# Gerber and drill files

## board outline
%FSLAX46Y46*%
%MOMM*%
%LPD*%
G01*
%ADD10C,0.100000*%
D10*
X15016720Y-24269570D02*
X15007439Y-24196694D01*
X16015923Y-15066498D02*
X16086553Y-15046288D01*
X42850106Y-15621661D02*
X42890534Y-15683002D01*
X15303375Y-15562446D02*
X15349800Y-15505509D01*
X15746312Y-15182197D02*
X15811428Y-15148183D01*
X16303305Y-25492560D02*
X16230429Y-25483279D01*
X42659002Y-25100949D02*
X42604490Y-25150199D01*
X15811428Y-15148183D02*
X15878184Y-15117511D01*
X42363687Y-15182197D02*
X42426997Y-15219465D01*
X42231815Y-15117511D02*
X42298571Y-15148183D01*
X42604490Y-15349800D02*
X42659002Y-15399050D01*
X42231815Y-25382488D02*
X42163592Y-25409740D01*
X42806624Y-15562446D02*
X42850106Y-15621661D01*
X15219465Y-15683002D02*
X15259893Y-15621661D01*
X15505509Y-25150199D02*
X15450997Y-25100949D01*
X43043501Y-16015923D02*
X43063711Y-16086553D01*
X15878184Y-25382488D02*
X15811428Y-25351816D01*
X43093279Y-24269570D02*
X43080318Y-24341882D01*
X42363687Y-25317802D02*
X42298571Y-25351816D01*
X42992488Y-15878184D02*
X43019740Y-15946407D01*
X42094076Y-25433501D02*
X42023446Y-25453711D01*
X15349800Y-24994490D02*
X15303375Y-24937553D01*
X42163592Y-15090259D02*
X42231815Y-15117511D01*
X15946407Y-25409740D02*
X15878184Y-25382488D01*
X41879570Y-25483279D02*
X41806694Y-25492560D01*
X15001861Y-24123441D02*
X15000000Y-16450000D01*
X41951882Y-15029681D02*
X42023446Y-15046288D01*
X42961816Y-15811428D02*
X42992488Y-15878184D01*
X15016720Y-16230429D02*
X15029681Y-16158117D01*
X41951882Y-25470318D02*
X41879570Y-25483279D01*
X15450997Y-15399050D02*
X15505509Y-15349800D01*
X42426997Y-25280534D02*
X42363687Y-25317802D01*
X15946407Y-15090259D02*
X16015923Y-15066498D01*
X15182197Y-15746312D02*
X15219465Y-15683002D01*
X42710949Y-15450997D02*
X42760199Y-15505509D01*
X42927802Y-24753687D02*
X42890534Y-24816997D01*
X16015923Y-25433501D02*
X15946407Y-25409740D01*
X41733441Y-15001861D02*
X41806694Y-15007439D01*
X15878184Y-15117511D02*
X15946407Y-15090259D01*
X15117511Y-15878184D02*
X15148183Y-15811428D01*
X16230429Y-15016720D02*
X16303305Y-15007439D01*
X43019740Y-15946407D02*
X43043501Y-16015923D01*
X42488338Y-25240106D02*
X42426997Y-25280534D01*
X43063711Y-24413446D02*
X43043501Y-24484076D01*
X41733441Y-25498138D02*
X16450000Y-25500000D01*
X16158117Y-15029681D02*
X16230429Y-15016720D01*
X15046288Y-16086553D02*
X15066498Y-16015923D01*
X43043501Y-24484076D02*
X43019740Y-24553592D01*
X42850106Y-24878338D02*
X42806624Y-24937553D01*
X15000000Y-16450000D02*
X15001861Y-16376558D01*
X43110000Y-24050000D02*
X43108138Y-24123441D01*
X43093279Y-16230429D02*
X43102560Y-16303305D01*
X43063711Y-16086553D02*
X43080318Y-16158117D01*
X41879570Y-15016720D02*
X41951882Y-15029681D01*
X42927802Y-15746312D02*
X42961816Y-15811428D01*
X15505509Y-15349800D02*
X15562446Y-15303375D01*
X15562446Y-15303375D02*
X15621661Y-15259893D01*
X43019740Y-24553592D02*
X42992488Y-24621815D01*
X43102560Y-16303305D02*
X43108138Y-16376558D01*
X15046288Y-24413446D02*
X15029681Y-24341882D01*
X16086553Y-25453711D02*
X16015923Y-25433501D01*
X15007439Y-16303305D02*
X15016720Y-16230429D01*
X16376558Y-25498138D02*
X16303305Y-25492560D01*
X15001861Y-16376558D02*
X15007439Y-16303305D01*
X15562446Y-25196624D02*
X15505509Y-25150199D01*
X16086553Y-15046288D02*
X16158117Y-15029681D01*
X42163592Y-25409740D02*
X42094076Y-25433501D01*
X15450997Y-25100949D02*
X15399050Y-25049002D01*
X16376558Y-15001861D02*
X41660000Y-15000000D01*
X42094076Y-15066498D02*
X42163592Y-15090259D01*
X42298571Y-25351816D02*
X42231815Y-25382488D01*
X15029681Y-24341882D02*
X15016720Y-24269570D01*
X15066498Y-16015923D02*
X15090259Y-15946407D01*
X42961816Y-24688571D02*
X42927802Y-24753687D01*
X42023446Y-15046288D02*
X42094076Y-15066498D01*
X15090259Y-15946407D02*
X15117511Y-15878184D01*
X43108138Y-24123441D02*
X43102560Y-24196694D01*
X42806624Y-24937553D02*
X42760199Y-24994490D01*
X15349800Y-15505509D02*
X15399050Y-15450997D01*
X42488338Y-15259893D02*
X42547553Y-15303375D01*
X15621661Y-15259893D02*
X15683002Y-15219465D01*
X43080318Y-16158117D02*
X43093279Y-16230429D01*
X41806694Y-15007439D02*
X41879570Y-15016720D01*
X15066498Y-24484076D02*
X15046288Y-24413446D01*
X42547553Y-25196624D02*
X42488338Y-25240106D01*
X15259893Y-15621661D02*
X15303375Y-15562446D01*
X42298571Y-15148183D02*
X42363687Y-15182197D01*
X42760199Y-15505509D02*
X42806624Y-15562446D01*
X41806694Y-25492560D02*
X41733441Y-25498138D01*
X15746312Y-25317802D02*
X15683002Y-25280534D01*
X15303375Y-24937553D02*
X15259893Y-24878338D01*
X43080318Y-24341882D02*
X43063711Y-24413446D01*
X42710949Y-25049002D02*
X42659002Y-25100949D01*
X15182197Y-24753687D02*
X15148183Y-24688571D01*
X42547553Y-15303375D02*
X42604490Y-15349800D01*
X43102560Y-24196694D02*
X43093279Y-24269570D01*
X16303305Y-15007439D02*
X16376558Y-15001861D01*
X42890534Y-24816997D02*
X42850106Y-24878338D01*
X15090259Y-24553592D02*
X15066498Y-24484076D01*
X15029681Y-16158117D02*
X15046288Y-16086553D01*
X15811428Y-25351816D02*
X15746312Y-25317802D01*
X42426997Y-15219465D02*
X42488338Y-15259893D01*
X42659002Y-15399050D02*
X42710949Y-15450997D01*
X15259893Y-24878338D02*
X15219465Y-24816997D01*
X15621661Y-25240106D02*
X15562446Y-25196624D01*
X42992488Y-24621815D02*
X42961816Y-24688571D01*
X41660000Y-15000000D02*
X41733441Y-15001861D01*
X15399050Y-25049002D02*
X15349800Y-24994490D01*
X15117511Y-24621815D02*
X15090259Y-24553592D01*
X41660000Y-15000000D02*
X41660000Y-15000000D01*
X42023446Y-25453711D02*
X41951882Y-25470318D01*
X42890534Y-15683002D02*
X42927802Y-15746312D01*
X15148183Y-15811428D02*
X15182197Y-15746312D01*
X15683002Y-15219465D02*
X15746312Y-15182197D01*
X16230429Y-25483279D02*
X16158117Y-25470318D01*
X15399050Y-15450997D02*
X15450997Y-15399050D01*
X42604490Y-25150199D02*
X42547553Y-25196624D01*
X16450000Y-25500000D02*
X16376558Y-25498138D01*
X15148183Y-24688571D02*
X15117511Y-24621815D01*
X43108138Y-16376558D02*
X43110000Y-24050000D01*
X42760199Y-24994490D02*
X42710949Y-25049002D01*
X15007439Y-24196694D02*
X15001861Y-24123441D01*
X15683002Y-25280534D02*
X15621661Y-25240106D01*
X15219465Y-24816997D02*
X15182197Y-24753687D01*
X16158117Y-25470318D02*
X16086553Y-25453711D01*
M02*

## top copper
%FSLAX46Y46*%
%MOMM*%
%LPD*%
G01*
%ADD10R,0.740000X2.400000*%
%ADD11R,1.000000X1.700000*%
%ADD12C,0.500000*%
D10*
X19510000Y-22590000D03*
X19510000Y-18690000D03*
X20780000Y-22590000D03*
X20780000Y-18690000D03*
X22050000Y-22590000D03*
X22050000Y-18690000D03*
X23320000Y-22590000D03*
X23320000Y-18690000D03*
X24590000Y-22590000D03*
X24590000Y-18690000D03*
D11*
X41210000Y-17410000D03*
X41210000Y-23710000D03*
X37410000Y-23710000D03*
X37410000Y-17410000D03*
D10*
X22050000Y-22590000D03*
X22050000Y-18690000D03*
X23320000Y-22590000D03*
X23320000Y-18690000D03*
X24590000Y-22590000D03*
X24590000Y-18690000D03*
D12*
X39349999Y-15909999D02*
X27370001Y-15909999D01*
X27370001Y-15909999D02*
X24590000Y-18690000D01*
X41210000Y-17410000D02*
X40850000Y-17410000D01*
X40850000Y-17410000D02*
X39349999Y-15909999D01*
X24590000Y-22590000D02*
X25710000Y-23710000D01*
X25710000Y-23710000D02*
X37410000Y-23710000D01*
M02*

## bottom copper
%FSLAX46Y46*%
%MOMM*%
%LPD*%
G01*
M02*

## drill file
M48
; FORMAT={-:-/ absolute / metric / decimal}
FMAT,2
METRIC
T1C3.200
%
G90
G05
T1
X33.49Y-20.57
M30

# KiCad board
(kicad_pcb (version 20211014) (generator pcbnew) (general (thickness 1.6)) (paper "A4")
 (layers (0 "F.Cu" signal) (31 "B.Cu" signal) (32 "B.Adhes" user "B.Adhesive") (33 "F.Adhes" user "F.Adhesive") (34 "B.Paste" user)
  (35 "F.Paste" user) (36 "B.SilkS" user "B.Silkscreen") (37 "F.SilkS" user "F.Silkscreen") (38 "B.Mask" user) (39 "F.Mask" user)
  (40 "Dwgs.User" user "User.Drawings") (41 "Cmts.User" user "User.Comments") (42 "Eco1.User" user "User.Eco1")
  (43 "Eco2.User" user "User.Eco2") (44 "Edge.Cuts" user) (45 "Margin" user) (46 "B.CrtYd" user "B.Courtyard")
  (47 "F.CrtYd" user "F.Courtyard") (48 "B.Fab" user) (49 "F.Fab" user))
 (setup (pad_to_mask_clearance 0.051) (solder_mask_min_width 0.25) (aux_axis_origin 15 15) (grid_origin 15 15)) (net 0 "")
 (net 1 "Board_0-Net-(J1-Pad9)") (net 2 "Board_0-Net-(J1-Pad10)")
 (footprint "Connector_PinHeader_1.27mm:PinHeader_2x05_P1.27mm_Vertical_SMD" (layer "F.Cu") (at 22.05 20.64 90)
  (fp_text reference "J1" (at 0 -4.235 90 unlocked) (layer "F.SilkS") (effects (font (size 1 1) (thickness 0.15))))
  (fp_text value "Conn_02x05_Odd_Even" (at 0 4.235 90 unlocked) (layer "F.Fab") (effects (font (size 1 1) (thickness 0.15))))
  (pad "1" smd rect locked (at -1.95 -2.54 90) (size 2.4 0.74) (layers "F.Cu" "F.Paste" "F.Mask"))
  (pad "2" smd rect locked (at 1.95 -2.54 90) (size 2.4 0.74) (layers "F.Cu" "F.Paste" "F.Mask"))
  (pad "3" smd rect locked (at -1.95 -1.27 90) (size 2.4 0.74) (layers "F.Cu" "F.Paste" "F.Mask"))
  (pad "4" smd rect locked (at 1.95 -1.27 90) (size 2.4 0.74) (layers "F.Cu" "F.Paste" "F.Mask"))
  (pad "5" smd rect locked (at -1.95 0 90) (size 2.4 0.74) (layers "F.Cu" "F.Paste" "F.Mask"))
  (pad "6" smd rect locked (at 1.95 0 90) (size 2.4 0.74) (layers "F.Cu" "F.Paste" "F.Mask"))
  (pad "7" smd rect locked (at -1.95 1.27 90) (size 2.4 0.74) (layers "F.Cu" "F.Paste" "F.Mask"))
  (pad "8" smd rect locked (at 1.95 1.27 90) (size 2.4 0.74) (layers "F.Cu" "F.Paste" "F.Mask"))
  (pad "9" smd rect locked (at -1.95 2.54 90) (size 2.4 0.74) (layers "F.Cu" "F.Paste" "F.Mask") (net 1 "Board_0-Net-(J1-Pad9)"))
  (pad "10" smd rect locked (at 1.95 2.54 90) (size 2.4 0.74) (layers "F.Cu" "F.Paste" "F.Mask") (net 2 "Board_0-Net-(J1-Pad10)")))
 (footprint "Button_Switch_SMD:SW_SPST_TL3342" (layer "F.Cu") (at 39.31 20.56 -90)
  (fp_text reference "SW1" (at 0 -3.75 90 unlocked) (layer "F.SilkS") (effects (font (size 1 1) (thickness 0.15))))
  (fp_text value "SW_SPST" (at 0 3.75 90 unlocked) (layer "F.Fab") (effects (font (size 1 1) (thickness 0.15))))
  (pad "1" smd rect locked (at -3.15 -1.9 270) (size 1.7 1) (layers "F.Cu" "F.Paste" "F.Mask") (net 2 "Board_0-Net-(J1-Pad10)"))
  (pad "1" smd rect locked (at 3.15 -1.9 270) (size 1.7 1) (layers "F.Cu" "F.Paste" "F.Mask") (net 2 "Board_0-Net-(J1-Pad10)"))
  (pad "2" smd rect locked (at 3.15 1.9 270) (size 1.7 1) (layers "F.Cu" "F.Paste" "F.Mask") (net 1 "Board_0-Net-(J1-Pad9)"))
  (pad "2" smd rect locked (at -3.15 1.9 270) (size 1.7 1) (layers "F.Cu" "F.Paste" "F.Mask") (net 1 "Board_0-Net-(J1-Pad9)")))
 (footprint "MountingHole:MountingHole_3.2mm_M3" (layer "F.Cu") (at 33.35 20.57 -90)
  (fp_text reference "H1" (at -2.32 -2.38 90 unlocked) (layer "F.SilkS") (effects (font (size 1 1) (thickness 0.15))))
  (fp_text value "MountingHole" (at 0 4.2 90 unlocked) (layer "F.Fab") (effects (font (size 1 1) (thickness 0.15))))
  (pad "" np_thru_hole circle locked (at 0 -0.14 270) (size 3.2 3.2) (drill 3.2) (layers *.Cu *.Mask)))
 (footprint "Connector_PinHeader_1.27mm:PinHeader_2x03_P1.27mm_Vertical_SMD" (layer "F.Cu") (at 23.32 20.64 90)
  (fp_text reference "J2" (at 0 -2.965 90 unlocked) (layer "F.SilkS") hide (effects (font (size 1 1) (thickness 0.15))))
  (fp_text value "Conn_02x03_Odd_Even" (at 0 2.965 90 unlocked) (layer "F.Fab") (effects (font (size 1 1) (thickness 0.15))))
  (pad "1" smd rect locked (at -1.95 -1.27 90) (size 2.4 0.74) (layers "F.Cu" "F.Paste" "F.Mask"))
  (pad "2" smd rect locked (at 1.95 -1.27 90) (size 2.4 0.74) (layers "F.Cu" "F.Paste" "F.Mask"))
  (pad "3" smd rect locked (at -1.95 0 90) (size 2.4 0.74) (layers "F.Cu" "F.Paste" "F.Mask"))
  (pad "4" smd rect locked (at 1.95 0 90) (size 2.4 0.74) (layers "F.Cu" "F.Paste" "F.Mask"))
  (pad "5" smd rect locked (at -1.95 1.27 90) (size 2.4 0.74) (layers "F.Cu" "F.Paste" "F.Mask") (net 1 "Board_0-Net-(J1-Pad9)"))
  (pad "6" smd rect locked (at 1.95 1.27 90) (size 2.4 0.74) (layers "F.Cu" "F.Paste" "F.Mask") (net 2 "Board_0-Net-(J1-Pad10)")))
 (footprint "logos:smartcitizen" (layer "B.Cu") (at 39.49 20.93)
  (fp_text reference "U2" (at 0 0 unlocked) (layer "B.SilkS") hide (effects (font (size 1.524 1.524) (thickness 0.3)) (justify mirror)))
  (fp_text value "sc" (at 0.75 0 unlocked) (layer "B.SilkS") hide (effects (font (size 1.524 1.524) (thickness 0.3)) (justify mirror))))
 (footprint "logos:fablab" (layer "B.Cu") (at 23.85 16.37)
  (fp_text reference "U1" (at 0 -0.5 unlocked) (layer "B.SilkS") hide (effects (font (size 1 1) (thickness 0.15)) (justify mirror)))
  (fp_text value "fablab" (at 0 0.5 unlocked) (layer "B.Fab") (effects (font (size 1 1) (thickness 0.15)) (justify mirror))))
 (gr_line (start 15.01672 24.26957) (end 15.007439 24.196694) (layer "Edge.Cuts") (width 0.1))
 (gr_line (start 16.015923 15.066498) (end 16.086553 15.046288) (layer "Edge.Cuts") (width 0.1))
 (gr_line (start 42.850106 15.621661) (end 42.890534 15.683002) (layer "Edge.Cuts") (width 0.1))
 (gr_line (start 15.303375 15.562446) (end 15.3498 15.505509) (layer "Edge.Cuts") (width 0.1))
 (gr_line (start 15.746312 15.182197) (end 15.811428 15.148183) (layer "Edge.Cuts") (width 0.1))
 (gr_line (start 16.303305 25.49256) (end 16.230429 25.483279) (layer "Edge.Cuts") (width 0.1))
 (gr_line (start 42.659002 25.100949) (end 42.60449 25.150199) (layer "Edge.Cuts") (width 0.1))
 (gr_line (start 15.811428 15.148183) (end 15.878184 15.117511) (layer "Edge.Cuts") (width 0.1))
 (gr_line (start 42.363687 15.182197) (end 42.426997 15.219465) (layer "Edge.Cuts") (width 0.1))
 (gr_line (start 42.231815 15.117511) (end 42.298571 15.148183) (layer "Edge.Cuts") (width 0.1))
 (gr_line (start 42.60449 15.3498) (end 42.659002 15.39905) (layer "Edge.Cuts") (width 0.1))
 (gr_line (start 42.231815 25.382488) (end 42.163592 25.40974) (layer "Edge.Cuts") (width 0.1))
 (gr_line (start 42.806624 15.562446) (end 42.850106 15.621661) (layer "Edge.Cuts") (width 0.1))
 (gr_line (start 15.219465 15.683002) (end 15.259893 15.621661) (layer "Edge.Cuts") (width 0.1))
 (gr_line (start 15.505509 25.150199) (end 15.450997 25.100949) (layer "Edge.Cuts") (width 0.1))
 (gr_line (start 43.043501 16.015923) (end 43.063711 16.086553) (layer "Edge.Cuts") (width 0.1))
 (gr_line (start 15.878184 25.382488) (end 15.811428 25.351816) (layer "Edge.Cuts") (width 0.1))
 (gr_line (start 43.093279 24.26957) (end 43.080318 24.341882) (layer "Edge.Cuts") (width 0.1))
 (gr_line (start 42.363687 25.317802) (end 42.298571 25.351816) (layer "Edge.Cuts") (width 0.1))
 (gr_line (start 42.992488 15.878184) (end 43.01974 15.946407) (layer "Edge.Cuts") (width 0.1))
 (gr_line (start 42.094076 25.433501) (end 42.023446 25.453711) (layer "Edge.Cuts") (width 0.1))
 (gr_line (start 15.3498 24.99449) (end 15.303375 24.937553) (layer "Edge.Cuts") (width 0.1))
 (gr_line (start 42.163592 15.090259) (end 42.231815 15.117511) (layer "Edge.Cuts") (width 0.1))
 (gr_line (start 15.946407 25.40974) (end 15.878184 25.382488) (layer "Edge.Cuts") (width 0.1))
 (gr_line (start 41.87957 25.483279) (end 41.806694 25.49256) (layer "Edge.Cuts") (width 0.1))
 (gr_line (start 15.001861 24.123441) (end 15 16.45) (layer "Edge.Cuts") (width 0.1))
 (gr_line (start 41.951882 15.029681) (end 42.023446 15.046288) (layer "Edge.Cuts") (width 0.1))
 (gr_line (start 42.961816 15.811428) (end 42.992488 15.878184) (layer "Edge.Cuts") (width 0.1))
 (gr_line (start 15.01672 16.230429) (end 15.029681 16.158117) (layer "Edge.Cuts") (width 0.1))
 (gr_line (start 41.951882 25.470318) (end 41.87957 25.483279) (layer "Edge.Cuts") (width 0.1))
 (gr_line (start 15.450997 15.39905) (end 15.505509 15.3498) (layer "Edge.Cuts") (width 0.1))
 (gr_line (start 42.426997 25.280534) (end 42.363687 25.317802) (layer "Edge.Cuts") (width 0.1))
 (gr_line (start 15.946407 15.090259) (end 16.015923 15.066498) (layer "Edge.Cuts") (width 0.1))
 (gr_line (start 15.182197 15.746312) (end 15.219465 15.683002) (layer "Edge.Cuts") (width 0.1))
 (gr_line (start 42.710949 15.450997) (end 42.760199 15.505509) (layer "Edge.Cuts") (width 0.1))
 (gr_line (start 42.927802 24.753687) (end 42.890534 24.816997) (layer "Edge.Cuts") (width 0.1))
 (gr_line (start 16.015923 25.433501) (end 15.946407 25.40974) (layer "Edge.Cuts") (width 0.1))
 (gr_line (start 41.733441 15.001861) (end 41.806694 15.007439) (layer "Edge.Cuts") (width 0.1))
 (gr_line (start 15.878184 15.117511) (end 15.946407 15.090259) (layer "Edge.Cuts") (width 0.1))
 (gr_line (start 15.117511 15.878184) (end 15.148183 15.811428) (layer "Edge.Cuts") (width 0.1))
 (gr_line (start 16.230429 15.01672) (end 16.303305 15.007439) (layer "Edge.Cuts") (width 0.1))
 (gr_line (start 43.01974 15.946407) (end 43.043501 16.015923) (layer "Edge.Cuts") (width 0.1))
 (gr_line (start 42.488338 25.240106) (end 42.426997 25.280534) (layer "Edge.Cuts") (width 0.1))
 (gr_line (start 43.063711 24.413446) (end 43.043501 24.484076) (layer "Edge.Cuts") (width 0.1))
 (gr_line (start 41.733441 25.498138) (end 16.45 25.5) (layer "Edge.Cuts") (width 0.1))
 (gr_line (start 16.158117 15.029681) (end 16.230429 15.01672) (layer "Edge.Cuts") (width 0.1))
 (gr_line (start 15.046288 16.086553) (end 15.066498 16.015923) (layer "Edge.Cuts") (width 0.1))
 (gr_line (start 43.043501 24.484076) (end 43.01974 24.553592) (layer "Edge.Cuts") (width 0.1))
 (gr_line (start 42.850106 24.878338) (end 42.806624 24.937553) (layer "Edge.Cuts") (width 0.1))
 (gr_line (start 15 16.45) (end 15.001861 16.376558) (layer "Edge.Cuts") (width 0.1))
 (gr_line (start 43.11 24.05) (end 43.108138 24.123441) (layer "Edge.Cuts") (width 0.1))
 (gr_line (start 43.093279 16.230429) (end 43.10256 16.303305) (layer "Edge.Cuts") (width 0.1))
 (gr_line (start 43.063711 16.086553) (end 43.080318 16.158117) (layer "Edge.Cuts") (width 0.1))
 (gr_line (start 41.87957 15.01672) (end 41.951882 15.029681) (layer "Edge.Cuts") (width 0.1))
 (gr_line (start 42.927802 15.746312) (end 42.961816 15.811428) (layer "Edge.Cuts") (width 0.1))
 (gr_line (start 15.505509 15.3498) (end 15.562446 15.303375) (layer "Edge.Cuts") (width 0.1))
 (gr_line (start 15.562446 15.303375) (end 15.621661 15.259893) (layer "Edge.Cuts") (width 0.1))
 (gr_line (start 43.01974 24.553592) (end 42.992488 24.621815) (layer "Edge.Cuts") (width 0.1))
 (gr_line (start 43.10256 16.303305) (end 43.108138 16.376558) (layer "Edge.Cuts") (width 0.1))
 (gr_line (start 15.046288 24.413446) (end 15.029681 24.341882) (layer "Edge.Cuts") (width 0.1))
 (gr_line (start 16.086553 25.453711) (end 16.015923 25.433501) (layer "Edge.Cuts") (width 0.1))
 (gr_line (start 15.007439 16.303305) (end 15.01672 16.230429) (layer "Edge.Cuts") (width 0.1))
 (gr_line (start 16.376558 25.498138) (end 16.303305 25.49256) (layer "Edge.Cuts") (width 0.1))
 (gr_line (start 15.001861 16.376558) (end 15.007439 16.303305) (layer "Edge.Cuts") (width 0.1))
 (gr_line (start 15.562446 25.196624) (end 15.505509 25.150199) (layer "Edge.Cuts") (width 0.1))
 (gr_line (start 16.086553 15.046288) (end 16.158117 15.029681) (layer "Edge.Cuts") (width 0.1))
 (gr_line (start 42.163592 25.40974) (end 42.094076 25.433501) (layer "Edge.Cuts") (width 0.1))
 (gr_line (start 15.450997 25.100949) (end 15.39905 25.049002) (layer "Edge.Cuts") (width 0.1))
 (gr_line (start 16.376558 15.001861) (end 41.66 15) (layer "Edge.Cuts") (width 0.1))
 (gr_line (start 42.094076 15.066498) (end 42.163592 15.090259) (layer "Edge.Cuts") (width 0.1))
 (gr_line (start 42.298571 25.351816) (end 42.231815 25.382488) (layer "Edge.Cuts") (width 0.1))
 (gr_line (start 15.029681 24.341882) (end 15.01672 24.26957) (layer "Edge.Cuts") (width 0.1))
 (gr_line (start 15.066498 16.015923) (end 15.090259 15.946407) (layer "Edge.Cuts") (width 0.1))
 (gr_line (start 42.961816 24.688571) (end 42.927802 24.753687) (layer "Edge.Cuts") (width 0.1))
 (gr_line (start 42.023446 15.046288) (end 42.094076 15.066498) (layer "Edge.Cuts") (width 0.1))
 (gr_line (start 15.090259 15.946407) (end 15.117511 15.878184) (layer "Edge.Cuts") (width 0.1))
 (gr_line (start 43.108138 24.123441) (end 43.10256 24.196694) (layer "Edge.Cuts") (width 0.1))
 (gr_line (start 42.806624 24.937553) (end 42.760199 24.99449) (layer "Edge.Cuts") (width 0.1))
 (gr_line (start 15.3498 15.505509) (end 15.39905 15.450997) (layer "Edge.Cuts") (width 0.1))
 (gr_line (start 42.488338 15.259893) (end 42.547553 15.303375) (layer "Edge.Cuts") (width 0.1))
 (gr_line (start 15.621661 15.259893) (end 15.683002 15.219465) (layer "Edge.Cuts") (width 0.1))
 (gr_line (start 43.080318 16.158117) (end 43.093279 16.230429) (layer "Edge.Cuts") (width 0.1))
 (gr_line (start 41.806694 15.007439) (end 41.87957 15.01672) (layer "Edge.Cuts") (width 0.1))
 (gr_line (start 15.066498 24.484076) (end 15.046288 24.413446) (layer "Edge.Cuts") (width 0.1))
 (gr_line (start 42.547553 25.196624) (end 42.488338 25.240106) (layer "Edge.Cuts") (width 0.1))
 (gr_line (start 15.259893 15.621661) (end 15.303375 15.562446) (layer "Edge.Cuts") (width 0.1))
 (gr_line (start 42.298571 15.148183) (end 42.363687 15.182197) (layer "Edge.Cuts") (width 0.1))
 (gr_line (start 42.760199 15.505509) (end 42.806624 15.562446) (layer "Edge.Cuts") (width 0.1))
 (gr_line (start 41.806694 25.49256) (end 41.733441 25.498138) (layer "Edge.Cuts") (width 0.1))
 (gr_line (start 15.746312 25.317802) (end 15.683002 25.280534) (layer "Edge.Cuts") (width 0.1))
 (gr_line (start 15.303375 24.937553) (end 15.259893 24.878338) (layer "Edge.Cuts") (width 0.1))
 (gr_line (start 43.080318 24.341882) (end 43.063711 24.413446) (layer "Edge.Cuts") (width 0.1))
 (gr_line (start 42.710949 25.049002) (end 42.659002 25.100949) (layer "Edge.Cuts") (width 0.1))
 (gr_line (start 15.182197 24.753687) (end 15.148183 24.688571) (layer "Edge.Cuts") (width 0.1))
 (gr_line (start 42.547553 15.303375) (end 42.60449 15.3498) (layer "Edge.Cuts") (width 0.1))
 (gr_line (start 43.10256 24.196694) (end 43.093279 24.26957) (layer "Edge.Cuts") (width 0.1))
 (gr_line (start 16.303305 15.007439) (end 16.376558 15.001861) (layer "Edge.Cuts") (width 0.1))
 (gr_line (start 42.890534 24.816997) (end 42.850106 24.878338) (layer "Edge.Cuts") (width 0.1))
 (gr_line (start 15.090259 24.553592) (end 15.066498 24.484076) (layer "Edge.Cuts") (width 0.1))
 (gr_line (start 15.029681 16.158117) (end 15.046288 16.086553) (layer "Edge.Cuts") (width 0.1))
 (gr_line (start 15.811428 25.351816) (end 15.746312 25.317802) (layer "Edge.Cuts") (width 0.1))
 (gr_line (start 42.426997 15.219465) (end 42.488338 15.259893) (layer "Edge.Cuts") (width 0.1))
 (gr_line (start 42.659002 15.39905) (end 42.710949 15.450997) (layer "Edge.Cuts") (width 0.1))
 (gr_line (start 15.259893 24.878338) (end 15.219465 24.816997) (layer "Edge.Cuts") (width 0.1))
 (gr_line (start 15.621661 25.240106) (end 15.562446 25.196624) (layer "Edge.Cuts") (width 0.1))
 (gr_line (start 42.992488 24.621815) (end 42.961816 24.688571) (layer "Edge.Cuts") (width 0.1))
 (gr_line (start 41.66 15) (end 41.733441 15.001861) (layer "Edge.Cuts") (width 0.1))
 (gr_line (start 15.39905 25.049002) (end 15.3498 24.99449) (layer "Edge.Cuts") (width 0.1))
 (gr_line (start 15.117511 24.621815) (end 15.090259 24.553592) (layer "Edge.Cuts") (width 0.1))
 (gr_line (start 41.66 15) (end 41.66 15) (layer "Edge.Cuts") (width 0.1))
 (gr_line (start 42.023446 25.453711) (end 41.951882 25.470318) (layer "Edge.Cuts") (width 0.1))
 (gr_line (start 42.890534 15.683002) (end 42.927802 15.746312) (layer "Edge.Cuts") (width 0.1))
 (gr_line (start 15.148183 15.811428) (end 15.182197 15.746312) (layer "Edge.Cuts") (width 0.1))
 (gr_line (start 15.683002 15.219465) (end 15.746312 15.182197) (layer "Edge.Cuts") (width 0.1))
 (gr_line (start 16.230429 25.483279) (end 16.158117 25.470318) (layer "Edge.Cuts") (width 0.1))
 (gr_line (start 15.39905 15.450997) (end 15.450997 15.39905) (layer "Edge.Cuts") (width 0.1))
 (gr_line (start 42.60449 25.150199) (end 42.547553 25.196624) (layer "Edge.Cuts") (width 0.1))
 (gr_line (start 16.45 25.5) (end 16.376558 25.498138) (layer "Edge.Cuts") (width 0.1))
 (gr_line (start 15.148183 24.688571) (end 15.117511 24.621815) (layer "Edge.Cuts") (width 0.1))
 (gr_line (start 43.108138 16.376558) (end 43.11 24.05) (layer "Edge.Cuts") (width 0.1))
 (gr_line (start 42.760199 24.99449) (end 42.710949 25.049002) (layer "Edge.Cuts") (width 0.1))
 (gr_line (start 15.007439 24.196694) (end 15.001861 24.123441) (layer "Edge.Cuts") (width 0.1))
 (gr_line (start 15.683002 25.280534) (end 15.621661 25.240106) (layer "Edge.Cuts") (width 0.1))
 (gr_line (start 15.219465 24.816997) (end 15.182197 24.753687) (layer "Edge.Cuts") (width 0.1))
 (gr_line (start 16.158117 25.470318) (end 16.086553 25.453711) (layer "Edge.Cuts") (width 0.1))
 (segment (start 39.349999 15.909999) (end 27.370001 15.909999) (width 0.5) (layer "F.Cu") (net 2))
 (segment (start 27.370001 15.909999) (end 24.59 18.69) (width 0.5) (layer "F.Cu") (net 2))
 (segment (start 41.21 17.41) (end 40.85 17.41) (width 0.5) (layer "F.Cu") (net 2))
 (segment (start 40.85 17.41) (end 39.349999 15.909999) (width 0.5) (layer "F.Cu") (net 2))
 (segment (start 24.59 22.59) (end 25.71 23.71) (width 0.5) (layer "F.Cu") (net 1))
 (segment (start 25.71 23.71) (end 37.41 23.71) (width 0.5) (layer "F.Cu") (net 1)))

